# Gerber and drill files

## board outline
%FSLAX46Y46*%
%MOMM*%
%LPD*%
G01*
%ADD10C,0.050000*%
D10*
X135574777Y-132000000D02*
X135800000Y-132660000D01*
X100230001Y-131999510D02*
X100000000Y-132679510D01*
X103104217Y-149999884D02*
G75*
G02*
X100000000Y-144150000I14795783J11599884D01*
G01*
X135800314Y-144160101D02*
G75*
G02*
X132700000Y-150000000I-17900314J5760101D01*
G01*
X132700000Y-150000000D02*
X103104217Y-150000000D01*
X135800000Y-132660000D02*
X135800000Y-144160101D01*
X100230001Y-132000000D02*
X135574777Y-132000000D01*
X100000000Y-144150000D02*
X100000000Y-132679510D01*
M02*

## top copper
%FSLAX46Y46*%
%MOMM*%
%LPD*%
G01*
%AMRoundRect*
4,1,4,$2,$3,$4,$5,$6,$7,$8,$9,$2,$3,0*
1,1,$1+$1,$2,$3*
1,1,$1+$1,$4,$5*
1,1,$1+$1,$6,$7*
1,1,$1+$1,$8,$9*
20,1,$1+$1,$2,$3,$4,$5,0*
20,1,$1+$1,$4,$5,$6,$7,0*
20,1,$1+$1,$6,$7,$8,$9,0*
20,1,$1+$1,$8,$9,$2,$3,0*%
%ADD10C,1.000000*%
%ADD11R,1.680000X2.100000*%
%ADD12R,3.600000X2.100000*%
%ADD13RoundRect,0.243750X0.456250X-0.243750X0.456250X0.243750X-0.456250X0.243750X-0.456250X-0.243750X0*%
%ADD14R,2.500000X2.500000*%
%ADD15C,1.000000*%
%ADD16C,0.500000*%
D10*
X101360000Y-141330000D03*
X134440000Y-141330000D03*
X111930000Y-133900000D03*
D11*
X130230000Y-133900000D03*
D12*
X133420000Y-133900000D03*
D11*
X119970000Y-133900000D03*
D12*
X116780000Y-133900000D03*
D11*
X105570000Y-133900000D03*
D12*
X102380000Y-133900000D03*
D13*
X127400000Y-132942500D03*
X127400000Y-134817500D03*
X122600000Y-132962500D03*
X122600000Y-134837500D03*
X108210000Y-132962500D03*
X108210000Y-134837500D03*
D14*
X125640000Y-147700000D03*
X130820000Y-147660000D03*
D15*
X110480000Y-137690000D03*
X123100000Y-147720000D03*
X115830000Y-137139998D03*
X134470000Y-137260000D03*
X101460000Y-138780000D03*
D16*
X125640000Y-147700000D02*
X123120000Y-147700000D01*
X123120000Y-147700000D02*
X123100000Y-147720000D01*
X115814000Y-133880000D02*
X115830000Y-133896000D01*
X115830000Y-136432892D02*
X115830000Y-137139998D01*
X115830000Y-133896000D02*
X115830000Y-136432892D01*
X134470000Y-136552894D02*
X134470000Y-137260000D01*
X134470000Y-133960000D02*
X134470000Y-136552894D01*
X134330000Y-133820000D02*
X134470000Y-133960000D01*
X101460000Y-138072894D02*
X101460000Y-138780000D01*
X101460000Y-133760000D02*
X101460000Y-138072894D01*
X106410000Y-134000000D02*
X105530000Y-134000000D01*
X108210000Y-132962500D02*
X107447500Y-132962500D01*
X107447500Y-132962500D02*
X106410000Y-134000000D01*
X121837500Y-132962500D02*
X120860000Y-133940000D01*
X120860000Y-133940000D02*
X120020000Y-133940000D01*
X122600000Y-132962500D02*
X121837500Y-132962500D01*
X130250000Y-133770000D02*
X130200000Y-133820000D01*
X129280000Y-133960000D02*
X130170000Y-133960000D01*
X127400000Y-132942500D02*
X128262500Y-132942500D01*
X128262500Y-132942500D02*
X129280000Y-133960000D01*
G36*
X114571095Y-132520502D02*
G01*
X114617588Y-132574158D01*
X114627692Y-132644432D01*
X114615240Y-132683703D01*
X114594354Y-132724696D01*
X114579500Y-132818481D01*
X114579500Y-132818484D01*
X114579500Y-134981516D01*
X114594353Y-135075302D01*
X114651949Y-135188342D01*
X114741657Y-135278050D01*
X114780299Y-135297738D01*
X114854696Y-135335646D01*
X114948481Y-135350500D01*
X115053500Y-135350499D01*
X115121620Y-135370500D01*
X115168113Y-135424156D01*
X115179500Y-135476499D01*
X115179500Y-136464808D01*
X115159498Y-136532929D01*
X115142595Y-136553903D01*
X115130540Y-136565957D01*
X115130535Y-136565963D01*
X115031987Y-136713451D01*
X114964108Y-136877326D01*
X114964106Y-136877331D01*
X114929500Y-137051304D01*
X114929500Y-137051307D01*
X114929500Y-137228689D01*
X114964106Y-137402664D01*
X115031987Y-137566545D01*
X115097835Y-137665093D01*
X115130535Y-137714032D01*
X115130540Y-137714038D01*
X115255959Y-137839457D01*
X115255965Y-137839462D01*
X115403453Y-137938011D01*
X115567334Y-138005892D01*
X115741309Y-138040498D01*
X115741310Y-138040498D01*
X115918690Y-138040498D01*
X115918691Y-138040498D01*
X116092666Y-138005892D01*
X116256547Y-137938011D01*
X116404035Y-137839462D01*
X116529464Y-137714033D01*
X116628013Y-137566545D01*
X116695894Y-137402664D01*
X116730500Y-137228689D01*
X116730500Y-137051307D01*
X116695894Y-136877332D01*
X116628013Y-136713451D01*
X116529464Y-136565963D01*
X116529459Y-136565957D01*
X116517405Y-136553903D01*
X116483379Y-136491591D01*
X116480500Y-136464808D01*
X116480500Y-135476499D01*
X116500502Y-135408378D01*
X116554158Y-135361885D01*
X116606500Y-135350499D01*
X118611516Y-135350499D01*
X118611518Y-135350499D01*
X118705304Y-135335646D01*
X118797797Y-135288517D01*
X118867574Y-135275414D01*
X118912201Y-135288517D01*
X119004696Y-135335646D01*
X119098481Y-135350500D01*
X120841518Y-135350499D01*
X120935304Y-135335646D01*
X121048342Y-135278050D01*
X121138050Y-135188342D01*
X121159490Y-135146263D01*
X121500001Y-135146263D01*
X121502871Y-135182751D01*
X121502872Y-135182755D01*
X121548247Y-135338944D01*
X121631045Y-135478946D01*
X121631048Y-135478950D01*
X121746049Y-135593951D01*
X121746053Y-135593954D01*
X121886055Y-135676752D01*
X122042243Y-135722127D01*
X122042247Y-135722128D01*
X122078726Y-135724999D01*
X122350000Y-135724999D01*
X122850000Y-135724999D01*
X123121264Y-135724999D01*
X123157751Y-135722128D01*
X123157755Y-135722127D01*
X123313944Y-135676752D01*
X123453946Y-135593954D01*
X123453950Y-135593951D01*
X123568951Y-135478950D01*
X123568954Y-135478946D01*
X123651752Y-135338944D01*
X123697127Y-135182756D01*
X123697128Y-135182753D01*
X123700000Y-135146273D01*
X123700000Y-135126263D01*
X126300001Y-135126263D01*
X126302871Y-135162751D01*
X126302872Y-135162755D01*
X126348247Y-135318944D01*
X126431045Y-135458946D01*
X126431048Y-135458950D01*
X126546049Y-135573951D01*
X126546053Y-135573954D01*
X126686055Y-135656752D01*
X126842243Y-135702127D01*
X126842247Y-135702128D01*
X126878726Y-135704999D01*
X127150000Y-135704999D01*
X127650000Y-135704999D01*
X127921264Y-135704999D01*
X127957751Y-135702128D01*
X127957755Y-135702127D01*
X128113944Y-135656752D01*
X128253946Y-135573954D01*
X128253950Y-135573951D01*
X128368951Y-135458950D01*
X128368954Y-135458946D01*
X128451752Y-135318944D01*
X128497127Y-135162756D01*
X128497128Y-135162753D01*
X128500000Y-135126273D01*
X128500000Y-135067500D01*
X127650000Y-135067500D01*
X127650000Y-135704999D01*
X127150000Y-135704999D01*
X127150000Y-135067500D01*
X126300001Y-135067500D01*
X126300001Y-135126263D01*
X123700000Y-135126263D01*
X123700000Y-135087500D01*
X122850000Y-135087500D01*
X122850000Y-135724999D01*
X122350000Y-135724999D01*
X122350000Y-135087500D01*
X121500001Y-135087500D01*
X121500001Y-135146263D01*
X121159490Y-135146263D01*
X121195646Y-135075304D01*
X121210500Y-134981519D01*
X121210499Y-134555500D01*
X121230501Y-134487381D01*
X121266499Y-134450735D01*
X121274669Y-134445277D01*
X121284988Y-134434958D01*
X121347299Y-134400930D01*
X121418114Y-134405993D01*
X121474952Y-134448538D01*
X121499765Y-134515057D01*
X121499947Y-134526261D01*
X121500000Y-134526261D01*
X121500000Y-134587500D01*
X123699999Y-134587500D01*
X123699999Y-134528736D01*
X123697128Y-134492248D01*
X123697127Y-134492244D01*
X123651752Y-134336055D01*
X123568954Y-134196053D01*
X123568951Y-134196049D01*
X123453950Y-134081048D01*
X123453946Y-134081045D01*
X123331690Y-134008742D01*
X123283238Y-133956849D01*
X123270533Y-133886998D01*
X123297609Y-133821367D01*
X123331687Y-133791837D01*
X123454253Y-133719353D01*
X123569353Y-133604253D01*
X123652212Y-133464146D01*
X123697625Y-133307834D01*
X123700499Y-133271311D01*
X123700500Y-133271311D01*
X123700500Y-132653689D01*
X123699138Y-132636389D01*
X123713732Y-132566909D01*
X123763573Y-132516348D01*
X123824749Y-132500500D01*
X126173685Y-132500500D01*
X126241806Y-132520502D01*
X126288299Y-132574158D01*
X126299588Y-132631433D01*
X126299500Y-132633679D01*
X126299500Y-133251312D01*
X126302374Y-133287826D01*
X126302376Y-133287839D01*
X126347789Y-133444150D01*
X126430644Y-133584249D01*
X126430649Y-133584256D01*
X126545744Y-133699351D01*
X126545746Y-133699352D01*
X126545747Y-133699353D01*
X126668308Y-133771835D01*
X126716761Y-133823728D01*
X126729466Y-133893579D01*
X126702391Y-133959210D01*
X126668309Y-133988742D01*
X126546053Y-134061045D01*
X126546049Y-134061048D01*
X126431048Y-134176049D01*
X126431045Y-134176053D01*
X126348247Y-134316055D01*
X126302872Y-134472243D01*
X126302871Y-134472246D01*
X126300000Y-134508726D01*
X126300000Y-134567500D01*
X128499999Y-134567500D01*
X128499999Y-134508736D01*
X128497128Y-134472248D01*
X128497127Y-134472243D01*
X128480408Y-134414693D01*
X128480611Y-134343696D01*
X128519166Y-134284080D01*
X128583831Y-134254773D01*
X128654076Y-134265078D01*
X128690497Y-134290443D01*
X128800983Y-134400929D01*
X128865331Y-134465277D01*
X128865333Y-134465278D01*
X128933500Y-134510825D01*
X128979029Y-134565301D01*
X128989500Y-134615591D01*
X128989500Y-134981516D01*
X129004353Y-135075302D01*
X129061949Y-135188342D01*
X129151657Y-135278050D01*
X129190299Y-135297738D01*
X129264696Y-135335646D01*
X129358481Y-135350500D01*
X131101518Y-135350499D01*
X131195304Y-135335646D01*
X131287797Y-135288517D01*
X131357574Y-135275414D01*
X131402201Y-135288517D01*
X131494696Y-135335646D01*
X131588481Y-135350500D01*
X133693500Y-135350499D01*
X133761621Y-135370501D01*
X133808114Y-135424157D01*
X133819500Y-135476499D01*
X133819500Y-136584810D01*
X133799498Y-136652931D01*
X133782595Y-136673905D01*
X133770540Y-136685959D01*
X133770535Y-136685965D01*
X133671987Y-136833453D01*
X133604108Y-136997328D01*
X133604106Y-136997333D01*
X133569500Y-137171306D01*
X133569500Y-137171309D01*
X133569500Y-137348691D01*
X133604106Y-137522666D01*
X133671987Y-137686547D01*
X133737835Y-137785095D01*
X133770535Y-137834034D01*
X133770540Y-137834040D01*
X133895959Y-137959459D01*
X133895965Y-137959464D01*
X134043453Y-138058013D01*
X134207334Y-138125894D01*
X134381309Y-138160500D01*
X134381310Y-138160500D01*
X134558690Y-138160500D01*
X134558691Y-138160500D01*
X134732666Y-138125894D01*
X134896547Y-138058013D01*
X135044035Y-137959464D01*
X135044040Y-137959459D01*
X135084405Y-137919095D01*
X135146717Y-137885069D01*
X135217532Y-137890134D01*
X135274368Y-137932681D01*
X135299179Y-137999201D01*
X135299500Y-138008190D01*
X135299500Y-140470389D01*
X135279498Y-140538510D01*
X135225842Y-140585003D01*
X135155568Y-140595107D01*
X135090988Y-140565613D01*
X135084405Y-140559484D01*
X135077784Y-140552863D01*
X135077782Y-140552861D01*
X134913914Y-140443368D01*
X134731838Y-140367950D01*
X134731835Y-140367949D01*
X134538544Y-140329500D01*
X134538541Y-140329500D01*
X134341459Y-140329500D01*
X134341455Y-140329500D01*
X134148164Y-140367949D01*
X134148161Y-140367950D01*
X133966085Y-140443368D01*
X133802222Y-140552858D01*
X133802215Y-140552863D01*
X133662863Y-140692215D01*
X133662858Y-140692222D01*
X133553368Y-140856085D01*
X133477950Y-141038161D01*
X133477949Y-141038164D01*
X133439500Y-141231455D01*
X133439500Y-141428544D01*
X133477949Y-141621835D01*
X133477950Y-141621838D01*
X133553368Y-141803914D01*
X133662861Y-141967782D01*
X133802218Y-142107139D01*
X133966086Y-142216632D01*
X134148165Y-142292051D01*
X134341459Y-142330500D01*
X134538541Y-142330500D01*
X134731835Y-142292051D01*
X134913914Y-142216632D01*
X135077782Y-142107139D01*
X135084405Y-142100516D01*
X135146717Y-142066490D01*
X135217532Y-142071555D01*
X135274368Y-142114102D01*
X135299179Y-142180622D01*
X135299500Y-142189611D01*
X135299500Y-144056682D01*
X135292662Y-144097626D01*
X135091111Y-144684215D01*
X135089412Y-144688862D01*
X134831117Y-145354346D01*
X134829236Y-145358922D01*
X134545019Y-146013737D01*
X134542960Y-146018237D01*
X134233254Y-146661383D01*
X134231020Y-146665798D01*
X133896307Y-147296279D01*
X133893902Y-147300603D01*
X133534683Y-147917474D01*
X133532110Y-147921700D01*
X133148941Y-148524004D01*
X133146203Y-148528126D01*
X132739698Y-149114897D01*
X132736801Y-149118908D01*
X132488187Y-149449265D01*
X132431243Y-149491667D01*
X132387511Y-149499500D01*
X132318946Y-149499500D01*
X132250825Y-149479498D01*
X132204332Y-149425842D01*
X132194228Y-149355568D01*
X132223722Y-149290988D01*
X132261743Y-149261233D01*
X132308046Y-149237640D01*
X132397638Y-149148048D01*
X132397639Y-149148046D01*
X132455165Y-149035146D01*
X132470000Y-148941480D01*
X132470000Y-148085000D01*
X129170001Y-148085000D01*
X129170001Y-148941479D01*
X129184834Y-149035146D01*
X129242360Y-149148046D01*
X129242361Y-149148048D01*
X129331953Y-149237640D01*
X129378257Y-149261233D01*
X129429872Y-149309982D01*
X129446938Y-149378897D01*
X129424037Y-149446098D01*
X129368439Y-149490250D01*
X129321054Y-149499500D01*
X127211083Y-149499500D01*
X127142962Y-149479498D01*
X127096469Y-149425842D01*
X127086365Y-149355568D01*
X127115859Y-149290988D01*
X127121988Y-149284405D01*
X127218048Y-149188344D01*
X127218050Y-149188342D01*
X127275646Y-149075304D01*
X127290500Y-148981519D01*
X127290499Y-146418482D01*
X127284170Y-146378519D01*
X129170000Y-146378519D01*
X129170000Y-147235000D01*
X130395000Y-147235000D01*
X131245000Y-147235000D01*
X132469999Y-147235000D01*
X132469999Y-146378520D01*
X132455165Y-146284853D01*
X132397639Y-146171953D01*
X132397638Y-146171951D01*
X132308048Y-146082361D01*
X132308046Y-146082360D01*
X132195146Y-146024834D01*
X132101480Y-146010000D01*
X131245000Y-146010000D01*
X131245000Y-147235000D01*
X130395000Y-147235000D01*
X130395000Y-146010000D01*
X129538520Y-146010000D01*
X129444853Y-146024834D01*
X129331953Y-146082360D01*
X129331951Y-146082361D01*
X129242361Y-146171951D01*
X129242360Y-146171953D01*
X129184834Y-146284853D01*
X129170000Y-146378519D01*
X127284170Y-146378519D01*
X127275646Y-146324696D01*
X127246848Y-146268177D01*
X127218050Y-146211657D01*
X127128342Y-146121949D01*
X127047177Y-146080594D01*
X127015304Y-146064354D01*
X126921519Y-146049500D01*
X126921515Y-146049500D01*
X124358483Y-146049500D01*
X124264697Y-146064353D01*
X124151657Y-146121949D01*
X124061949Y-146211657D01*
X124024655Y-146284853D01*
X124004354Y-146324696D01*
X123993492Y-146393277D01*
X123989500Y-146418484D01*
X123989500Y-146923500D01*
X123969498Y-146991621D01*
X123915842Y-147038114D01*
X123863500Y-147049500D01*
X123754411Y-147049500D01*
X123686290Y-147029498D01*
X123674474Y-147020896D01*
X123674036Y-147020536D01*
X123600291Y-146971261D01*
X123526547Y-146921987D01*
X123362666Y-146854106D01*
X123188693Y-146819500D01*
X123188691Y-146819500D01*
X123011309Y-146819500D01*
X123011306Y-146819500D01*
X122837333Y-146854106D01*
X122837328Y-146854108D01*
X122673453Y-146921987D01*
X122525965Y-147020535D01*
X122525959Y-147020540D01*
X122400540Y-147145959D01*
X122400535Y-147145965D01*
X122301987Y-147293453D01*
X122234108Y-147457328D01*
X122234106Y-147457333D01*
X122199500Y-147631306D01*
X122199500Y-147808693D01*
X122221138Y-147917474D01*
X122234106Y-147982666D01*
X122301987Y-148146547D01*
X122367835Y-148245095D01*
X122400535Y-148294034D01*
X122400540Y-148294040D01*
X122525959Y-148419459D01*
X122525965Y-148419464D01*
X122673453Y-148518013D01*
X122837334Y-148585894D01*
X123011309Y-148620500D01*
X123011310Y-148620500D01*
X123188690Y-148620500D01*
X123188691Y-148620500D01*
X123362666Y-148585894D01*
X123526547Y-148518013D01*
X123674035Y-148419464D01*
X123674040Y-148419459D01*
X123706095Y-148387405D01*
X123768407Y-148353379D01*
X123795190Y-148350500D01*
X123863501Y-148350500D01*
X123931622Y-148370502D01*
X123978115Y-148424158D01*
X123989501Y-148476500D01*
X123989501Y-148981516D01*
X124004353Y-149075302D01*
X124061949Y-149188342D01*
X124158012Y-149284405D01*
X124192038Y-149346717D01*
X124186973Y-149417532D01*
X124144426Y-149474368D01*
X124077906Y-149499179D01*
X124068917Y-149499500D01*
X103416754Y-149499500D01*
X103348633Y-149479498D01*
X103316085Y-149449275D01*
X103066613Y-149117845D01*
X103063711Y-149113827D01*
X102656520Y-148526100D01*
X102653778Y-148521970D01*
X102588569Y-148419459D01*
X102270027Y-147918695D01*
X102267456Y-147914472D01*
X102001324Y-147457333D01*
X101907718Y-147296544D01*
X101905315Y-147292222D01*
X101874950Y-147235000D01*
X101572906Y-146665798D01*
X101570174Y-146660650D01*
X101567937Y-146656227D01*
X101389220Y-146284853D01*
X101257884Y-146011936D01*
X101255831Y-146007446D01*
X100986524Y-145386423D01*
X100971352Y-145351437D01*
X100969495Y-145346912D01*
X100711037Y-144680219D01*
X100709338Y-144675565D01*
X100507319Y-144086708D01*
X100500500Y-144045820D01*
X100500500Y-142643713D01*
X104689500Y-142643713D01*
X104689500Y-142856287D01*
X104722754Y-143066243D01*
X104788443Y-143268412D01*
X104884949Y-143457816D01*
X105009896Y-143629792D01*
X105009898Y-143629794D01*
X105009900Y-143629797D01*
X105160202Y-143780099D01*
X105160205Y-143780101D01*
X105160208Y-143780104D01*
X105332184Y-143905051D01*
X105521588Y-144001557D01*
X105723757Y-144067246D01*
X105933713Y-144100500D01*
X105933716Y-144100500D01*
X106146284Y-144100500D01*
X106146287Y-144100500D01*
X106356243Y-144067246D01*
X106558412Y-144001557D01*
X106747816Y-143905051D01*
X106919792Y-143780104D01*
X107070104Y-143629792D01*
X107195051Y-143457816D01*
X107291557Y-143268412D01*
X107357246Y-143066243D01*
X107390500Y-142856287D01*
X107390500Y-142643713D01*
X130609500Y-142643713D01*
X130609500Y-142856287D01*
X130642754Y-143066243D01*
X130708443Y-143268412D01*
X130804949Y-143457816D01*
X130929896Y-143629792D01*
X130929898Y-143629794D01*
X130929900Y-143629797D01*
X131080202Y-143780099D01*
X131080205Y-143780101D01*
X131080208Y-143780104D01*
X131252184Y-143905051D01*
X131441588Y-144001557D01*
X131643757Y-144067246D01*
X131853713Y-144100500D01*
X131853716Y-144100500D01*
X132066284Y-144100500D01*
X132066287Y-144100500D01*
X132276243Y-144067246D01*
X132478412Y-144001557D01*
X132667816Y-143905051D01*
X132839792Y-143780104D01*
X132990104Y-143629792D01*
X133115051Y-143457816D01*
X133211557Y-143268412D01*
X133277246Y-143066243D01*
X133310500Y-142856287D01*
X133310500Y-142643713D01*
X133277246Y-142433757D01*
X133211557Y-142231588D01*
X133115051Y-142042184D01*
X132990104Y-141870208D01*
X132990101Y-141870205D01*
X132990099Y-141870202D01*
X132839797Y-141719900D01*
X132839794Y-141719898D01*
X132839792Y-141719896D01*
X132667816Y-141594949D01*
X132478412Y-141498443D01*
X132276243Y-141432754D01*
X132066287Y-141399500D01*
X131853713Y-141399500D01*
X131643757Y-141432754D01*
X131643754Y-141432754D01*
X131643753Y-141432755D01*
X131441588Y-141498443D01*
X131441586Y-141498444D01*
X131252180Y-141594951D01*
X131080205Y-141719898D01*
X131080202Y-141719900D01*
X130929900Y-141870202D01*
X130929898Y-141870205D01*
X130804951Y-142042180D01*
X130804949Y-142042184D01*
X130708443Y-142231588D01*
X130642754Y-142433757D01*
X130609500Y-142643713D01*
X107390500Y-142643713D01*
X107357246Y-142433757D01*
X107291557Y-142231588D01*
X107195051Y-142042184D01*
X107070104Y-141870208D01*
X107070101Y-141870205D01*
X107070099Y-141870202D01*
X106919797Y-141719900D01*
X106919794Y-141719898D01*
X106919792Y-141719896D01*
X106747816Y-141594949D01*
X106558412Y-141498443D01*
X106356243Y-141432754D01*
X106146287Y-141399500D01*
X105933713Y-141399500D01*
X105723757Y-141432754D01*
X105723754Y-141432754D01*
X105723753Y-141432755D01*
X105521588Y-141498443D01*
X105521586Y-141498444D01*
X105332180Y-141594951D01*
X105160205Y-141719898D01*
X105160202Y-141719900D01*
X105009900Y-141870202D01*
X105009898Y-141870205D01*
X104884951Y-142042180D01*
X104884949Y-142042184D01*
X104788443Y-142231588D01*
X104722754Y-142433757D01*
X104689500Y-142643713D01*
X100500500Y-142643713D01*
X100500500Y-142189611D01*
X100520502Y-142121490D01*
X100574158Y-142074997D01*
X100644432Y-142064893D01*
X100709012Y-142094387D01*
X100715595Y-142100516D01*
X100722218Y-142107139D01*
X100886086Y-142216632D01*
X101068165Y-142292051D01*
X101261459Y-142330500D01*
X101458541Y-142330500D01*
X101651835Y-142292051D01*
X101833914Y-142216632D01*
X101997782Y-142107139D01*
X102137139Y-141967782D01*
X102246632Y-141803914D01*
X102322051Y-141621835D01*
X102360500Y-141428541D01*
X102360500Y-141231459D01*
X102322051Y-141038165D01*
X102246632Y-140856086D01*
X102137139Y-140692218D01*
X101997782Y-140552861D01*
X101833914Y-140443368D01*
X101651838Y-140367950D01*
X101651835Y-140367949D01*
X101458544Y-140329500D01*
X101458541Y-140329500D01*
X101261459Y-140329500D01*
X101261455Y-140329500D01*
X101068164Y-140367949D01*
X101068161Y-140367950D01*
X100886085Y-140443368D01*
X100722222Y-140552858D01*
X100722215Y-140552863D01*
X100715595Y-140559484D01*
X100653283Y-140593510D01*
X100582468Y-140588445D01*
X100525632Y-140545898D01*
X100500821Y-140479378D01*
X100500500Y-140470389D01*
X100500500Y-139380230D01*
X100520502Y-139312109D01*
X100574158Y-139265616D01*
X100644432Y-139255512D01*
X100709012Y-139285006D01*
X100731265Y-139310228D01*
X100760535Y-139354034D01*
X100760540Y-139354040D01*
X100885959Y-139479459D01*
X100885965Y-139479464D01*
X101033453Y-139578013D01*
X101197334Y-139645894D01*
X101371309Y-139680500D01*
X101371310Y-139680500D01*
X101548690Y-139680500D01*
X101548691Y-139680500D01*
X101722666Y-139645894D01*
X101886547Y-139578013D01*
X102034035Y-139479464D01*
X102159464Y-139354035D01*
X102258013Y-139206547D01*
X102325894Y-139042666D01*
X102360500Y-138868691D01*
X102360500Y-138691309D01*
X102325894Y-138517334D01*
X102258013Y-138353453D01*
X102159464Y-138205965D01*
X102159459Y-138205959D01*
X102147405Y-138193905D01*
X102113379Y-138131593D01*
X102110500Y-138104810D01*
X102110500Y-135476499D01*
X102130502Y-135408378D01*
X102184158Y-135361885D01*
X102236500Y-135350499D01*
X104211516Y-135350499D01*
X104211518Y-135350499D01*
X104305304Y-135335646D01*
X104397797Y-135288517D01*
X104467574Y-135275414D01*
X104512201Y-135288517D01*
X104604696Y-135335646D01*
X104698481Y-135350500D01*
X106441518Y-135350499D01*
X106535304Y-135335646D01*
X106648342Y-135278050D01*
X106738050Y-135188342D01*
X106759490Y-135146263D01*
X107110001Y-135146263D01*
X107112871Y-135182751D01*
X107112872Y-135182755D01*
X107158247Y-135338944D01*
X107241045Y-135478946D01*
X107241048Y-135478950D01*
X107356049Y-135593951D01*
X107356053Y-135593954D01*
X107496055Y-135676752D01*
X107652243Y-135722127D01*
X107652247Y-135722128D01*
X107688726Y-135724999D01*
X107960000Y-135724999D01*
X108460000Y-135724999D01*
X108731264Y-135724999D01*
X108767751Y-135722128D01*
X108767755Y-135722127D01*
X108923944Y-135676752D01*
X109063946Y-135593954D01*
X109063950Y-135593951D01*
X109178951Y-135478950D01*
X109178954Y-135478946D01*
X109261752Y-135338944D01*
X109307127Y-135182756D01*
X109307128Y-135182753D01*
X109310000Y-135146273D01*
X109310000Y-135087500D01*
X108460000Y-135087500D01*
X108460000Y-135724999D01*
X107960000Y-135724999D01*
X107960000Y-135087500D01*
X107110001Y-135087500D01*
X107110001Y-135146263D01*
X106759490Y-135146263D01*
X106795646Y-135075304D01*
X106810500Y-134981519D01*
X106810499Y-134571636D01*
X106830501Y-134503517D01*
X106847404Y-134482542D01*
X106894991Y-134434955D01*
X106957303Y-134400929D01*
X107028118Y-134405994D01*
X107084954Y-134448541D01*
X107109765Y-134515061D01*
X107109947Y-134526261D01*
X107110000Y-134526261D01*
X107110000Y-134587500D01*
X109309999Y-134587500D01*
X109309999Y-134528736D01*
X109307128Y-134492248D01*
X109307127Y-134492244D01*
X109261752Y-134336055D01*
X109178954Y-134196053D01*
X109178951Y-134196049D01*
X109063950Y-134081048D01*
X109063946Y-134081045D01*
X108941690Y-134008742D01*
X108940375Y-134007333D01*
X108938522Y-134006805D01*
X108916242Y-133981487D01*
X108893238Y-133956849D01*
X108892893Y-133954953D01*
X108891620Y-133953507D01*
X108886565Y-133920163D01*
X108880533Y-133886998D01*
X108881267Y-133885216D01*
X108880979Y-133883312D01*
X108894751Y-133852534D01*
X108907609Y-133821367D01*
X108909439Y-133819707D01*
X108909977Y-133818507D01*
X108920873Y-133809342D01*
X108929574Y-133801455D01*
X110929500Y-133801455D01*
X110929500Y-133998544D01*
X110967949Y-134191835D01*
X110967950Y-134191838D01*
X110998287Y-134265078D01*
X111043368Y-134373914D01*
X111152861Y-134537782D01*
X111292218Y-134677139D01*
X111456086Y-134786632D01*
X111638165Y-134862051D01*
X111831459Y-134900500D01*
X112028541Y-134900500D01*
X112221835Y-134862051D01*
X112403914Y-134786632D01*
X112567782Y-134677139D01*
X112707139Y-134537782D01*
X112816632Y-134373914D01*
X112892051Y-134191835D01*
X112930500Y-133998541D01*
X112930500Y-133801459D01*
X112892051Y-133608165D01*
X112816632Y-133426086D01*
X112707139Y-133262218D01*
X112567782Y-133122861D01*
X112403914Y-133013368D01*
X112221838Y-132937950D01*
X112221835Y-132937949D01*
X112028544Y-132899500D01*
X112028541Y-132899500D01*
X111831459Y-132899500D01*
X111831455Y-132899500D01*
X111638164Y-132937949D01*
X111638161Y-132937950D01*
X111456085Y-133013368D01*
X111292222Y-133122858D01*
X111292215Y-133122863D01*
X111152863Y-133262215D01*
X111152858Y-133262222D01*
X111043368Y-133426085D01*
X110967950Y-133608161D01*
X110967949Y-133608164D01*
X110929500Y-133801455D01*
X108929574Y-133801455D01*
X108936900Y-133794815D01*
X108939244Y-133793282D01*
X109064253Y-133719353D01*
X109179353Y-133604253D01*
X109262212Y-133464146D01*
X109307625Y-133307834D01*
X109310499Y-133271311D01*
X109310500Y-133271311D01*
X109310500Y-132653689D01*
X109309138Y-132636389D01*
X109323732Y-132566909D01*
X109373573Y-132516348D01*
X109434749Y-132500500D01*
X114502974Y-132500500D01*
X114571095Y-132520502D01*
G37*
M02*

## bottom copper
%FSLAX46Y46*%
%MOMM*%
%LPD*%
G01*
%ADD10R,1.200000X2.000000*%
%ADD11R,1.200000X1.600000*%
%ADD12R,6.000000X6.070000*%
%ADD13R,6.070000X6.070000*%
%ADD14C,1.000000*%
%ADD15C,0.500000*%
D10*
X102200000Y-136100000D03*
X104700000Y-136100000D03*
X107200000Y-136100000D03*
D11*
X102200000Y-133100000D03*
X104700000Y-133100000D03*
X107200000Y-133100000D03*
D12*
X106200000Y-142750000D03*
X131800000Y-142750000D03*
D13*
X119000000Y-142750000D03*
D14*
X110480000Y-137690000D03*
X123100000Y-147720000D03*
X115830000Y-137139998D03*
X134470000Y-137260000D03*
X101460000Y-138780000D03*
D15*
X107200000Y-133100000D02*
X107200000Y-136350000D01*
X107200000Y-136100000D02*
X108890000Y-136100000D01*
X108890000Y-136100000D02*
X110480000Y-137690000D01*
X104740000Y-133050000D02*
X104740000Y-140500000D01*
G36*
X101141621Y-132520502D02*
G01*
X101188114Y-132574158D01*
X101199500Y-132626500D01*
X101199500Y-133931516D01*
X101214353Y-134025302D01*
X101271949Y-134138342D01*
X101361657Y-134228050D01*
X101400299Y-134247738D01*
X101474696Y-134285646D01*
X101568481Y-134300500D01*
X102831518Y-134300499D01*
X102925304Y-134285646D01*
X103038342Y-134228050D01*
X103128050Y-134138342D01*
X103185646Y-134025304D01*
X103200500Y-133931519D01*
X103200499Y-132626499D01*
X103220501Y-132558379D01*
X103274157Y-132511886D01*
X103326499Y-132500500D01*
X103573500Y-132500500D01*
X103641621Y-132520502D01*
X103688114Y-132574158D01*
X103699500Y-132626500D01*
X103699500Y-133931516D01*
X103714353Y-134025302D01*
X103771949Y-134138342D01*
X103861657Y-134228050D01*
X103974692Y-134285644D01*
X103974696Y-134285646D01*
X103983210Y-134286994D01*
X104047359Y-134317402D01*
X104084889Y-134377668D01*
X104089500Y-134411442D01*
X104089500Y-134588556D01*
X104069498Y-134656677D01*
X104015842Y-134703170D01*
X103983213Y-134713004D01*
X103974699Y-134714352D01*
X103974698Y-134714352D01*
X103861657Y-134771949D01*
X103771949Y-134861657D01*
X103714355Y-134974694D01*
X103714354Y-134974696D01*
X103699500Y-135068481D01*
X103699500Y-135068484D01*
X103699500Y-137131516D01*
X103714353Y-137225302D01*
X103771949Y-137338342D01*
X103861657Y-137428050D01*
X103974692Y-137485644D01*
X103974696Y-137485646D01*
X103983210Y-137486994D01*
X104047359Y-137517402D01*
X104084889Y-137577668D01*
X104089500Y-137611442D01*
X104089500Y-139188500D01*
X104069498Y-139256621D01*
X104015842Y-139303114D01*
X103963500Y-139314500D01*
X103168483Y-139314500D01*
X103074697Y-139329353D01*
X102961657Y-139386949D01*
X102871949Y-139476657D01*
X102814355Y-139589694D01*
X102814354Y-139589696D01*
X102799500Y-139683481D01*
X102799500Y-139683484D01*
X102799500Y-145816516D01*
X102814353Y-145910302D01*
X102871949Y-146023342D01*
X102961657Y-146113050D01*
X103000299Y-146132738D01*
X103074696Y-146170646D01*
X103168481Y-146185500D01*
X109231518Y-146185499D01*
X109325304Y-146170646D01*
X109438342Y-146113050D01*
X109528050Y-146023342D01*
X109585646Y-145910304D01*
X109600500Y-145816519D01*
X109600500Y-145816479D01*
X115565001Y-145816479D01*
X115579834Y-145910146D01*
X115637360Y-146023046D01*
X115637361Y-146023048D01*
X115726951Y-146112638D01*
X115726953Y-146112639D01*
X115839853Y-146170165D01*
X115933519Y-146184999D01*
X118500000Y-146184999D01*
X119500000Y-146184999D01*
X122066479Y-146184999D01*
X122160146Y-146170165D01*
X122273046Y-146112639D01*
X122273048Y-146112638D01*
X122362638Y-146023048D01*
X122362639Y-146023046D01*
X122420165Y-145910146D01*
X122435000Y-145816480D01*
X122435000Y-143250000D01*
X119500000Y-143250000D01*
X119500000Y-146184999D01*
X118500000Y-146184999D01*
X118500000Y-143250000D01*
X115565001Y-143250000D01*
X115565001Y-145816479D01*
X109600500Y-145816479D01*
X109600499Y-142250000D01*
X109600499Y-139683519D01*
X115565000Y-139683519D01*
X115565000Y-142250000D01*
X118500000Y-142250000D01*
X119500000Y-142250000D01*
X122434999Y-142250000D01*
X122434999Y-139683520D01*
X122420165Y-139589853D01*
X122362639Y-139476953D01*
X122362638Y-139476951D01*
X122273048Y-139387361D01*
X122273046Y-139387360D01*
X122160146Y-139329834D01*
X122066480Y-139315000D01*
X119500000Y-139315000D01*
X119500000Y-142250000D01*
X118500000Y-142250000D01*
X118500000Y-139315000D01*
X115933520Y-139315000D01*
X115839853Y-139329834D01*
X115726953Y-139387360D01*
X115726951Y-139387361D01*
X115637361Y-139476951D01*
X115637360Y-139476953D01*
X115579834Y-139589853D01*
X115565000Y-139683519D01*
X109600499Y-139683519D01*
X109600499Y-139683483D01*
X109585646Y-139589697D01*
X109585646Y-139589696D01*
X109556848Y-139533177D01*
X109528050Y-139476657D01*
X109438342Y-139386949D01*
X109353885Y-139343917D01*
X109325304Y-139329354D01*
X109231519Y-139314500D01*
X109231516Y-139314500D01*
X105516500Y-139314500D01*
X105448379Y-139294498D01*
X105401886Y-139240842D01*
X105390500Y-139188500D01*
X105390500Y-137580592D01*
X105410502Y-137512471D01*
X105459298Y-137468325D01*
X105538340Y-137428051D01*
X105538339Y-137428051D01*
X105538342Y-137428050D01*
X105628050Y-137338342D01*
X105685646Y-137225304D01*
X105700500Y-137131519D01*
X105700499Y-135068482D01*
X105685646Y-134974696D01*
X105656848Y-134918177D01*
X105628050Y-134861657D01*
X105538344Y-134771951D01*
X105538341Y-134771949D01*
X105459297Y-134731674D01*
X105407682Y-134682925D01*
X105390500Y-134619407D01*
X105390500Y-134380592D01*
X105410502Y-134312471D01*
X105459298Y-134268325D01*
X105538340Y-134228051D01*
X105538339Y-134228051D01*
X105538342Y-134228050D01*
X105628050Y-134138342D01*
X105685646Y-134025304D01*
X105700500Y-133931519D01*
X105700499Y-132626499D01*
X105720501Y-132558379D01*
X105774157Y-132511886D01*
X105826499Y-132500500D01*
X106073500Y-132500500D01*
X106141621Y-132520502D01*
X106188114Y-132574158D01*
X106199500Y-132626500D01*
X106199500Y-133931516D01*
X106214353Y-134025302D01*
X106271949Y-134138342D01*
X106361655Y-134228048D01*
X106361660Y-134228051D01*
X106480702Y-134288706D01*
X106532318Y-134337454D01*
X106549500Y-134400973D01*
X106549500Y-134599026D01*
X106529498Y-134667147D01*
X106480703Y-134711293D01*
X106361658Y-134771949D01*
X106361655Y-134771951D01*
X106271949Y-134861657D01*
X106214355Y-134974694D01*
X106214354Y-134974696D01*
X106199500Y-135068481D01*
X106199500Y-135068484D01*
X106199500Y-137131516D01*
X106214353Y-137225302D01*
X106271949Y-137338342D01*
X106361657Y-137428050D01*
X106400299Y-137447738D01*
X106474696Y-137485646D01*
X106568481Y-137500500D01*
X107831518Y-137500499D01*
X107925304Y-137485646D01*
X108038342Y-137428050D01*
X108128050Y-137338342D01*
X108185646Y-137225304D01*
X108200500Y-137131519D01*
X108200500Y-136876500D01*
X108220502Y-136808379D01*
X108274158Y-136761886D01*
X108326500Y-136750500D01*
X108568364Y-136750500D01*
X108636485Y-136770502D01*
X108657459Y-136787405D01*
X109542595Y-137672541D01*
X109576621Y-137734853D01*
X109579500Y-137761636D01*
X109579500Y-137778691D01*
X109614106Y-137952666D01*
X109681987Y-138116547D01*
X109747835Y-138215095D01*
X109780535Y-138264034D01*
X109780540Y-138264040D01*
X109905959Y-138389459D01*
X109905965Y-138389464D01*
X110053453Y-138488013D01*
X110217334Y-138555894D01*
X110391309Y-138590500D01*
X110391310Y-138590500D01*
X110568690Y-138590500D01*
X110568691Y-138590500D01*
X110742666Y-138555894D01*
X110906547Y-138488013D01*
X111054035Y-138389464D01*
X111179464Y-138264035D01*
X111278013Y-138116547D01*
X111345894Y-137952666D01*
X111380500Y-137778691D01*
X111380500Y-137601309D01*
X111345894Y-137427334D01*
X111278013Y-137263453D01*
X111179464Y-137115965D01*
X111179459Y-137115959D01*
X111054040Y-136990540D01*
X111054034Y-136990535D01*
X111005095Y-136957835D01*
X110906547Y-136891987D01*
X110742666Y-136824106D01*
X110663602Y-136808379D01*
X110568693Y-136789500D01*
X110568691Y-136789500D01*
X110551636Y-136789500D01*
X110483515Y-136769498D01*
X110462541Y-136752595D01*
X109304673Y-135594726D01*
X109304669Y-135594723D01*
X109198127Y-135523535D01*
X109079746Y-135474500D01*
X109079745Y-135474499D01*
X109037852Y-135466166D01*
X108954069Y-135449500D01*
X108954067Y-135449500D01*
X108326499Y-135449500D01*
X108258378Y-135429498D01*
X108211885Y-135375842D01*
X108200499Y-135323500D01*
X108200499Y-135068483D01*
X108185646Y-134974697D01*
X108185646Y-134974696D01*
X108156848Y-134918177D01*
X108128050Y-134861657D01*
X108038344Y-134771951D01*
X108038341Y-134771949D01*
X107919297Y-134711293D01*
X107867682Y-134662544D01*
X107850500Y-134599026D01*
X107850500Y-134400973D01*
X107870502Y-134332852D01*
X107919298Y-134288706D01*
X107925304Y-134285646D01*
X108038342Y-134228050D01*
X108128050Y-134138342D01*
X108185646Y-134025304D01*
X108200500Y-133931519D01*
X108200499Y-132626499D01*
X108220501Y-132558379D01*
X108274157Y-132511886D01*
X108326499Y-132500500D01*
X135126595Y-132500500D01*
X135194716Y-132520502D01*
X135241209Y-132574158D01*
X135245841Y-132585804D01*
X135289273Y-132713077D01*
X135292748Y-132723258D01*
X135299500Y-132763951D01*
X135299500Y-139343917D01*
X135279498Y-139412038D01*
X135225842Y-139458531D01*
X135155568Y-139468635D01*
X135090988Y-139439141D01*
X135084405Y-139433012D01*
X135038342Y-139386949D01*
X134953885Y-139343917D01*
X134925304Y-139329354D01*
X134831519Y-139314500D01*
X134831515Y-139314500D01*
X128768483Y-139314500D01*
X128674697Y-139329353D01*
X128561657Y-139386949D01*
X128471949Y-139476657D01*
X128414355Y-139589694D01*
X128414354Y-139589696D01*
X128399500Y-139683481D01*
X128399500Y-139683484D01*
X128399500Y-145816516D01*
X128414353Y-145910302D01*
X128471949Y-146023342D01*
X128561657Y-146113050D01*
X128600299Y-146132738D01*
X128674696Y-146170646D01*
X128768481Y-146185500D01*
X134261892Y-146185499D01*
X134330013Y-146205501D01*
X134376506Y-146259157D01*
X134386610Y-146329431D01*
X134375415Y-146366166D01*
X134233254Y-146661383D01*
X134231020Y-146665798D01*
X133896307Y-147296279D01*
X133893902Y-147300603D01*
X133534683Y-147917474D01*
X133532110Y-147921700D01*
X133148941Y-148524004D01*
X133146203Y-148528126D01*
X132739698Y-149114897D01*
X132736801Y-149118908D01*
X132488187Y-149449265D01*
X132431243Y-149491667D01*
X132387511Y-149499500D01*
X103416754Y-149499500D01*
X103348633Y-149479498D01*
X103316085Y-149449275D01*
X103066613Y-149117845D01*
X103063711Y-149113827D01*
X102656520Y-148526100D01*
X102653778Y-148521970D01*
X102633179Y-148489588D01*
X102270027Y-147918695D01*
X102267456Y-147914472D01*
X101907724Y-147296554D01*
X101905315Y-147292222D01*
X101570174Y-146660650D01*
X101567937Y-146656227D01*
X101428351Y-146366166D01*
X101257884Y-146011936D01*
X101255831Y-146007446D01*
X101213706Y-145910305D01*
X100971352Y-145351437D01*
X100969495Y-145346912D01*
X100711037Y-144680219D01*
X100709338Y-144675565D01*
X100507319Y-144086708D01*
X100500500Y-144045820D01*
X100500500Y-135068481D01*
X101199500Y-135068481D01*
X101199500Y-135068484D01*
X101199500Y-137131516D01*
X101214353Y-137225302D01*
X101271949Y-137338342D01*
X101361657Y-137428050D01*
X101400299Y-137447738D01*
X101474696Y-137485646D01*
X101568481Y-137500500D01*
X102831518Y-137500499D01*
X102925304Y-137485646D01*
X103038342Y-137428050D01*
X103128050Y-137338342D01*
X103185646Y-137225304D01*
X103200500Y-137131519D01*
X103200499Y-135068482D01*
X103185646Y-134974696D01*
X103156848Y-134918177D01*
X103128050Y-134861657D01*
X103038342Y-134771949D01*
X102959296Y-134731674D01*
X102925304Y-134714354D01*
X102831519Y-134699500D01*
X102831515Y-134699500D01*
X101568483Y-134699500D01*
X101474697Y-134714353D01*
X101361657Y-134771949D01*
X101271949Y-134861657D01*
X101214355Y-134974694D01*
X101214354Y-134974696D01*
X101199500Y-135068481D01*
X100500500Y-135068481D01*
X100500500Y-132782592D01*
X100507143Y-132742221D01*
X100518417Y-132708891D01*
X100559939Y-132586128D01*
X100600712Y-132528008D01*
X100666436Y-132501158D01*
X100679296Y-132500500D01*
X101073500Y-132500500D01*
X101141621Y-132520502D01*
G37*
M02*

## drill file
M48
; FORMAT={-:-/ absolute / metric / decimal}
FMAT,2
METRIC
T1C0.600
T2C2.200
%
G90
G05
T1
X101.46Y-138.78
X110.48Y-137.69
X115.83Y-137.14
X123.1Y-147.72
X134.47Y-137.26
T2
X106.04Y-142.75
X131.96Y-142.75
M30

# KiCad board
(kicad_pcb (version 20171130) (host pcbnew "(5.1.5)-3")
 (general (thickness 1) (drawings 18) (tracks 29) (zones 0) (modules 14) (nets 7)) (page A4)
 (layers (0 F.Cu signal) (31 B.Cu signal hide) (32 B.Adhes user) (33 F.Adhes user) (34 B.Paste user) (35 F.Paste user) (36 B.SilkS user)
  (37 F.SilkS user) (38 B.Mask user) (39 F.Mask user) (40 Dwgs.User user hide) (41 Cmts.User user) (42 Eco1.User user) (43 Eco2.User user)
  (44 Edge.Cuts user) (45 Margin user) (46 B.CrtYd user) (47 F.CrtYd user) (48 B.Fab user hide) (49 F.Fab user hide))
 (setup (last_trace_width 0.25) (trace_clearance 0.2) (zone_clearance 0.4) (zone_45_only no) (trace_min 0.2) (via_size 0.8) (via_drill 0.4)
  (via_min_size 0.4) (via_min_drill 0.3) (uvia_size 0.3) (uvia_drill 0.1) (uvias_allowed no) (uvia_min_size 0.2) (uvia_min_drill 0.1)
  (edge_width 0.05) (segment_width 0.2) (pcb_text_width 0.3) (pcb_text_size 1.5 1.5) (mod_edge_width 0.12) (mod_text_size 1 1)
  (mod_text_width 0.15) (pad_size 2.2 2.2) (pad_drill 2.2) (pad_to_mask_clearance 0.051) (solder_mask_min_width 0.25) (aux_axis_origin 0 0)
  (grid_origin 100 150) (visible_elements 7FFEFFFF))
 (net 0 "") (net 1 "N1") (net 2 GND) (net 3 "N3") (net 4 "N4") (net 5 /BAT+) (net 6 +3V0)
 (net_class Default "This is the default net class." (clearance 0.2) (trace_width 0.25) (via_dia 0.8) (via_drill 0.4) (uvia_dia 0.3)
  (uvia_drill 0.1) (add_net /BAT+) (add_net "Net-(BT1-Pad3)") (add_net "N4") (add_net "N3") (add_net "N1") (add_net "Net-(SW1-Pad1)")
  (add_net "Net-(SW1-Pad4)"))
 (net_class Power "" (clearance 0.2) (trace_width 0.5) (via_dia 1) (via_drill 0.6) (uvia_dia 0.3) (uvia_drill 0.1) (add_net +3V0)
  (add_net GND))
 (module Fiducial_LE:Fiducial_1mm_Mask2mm (layer F.Cu) (at 101.36 141.33)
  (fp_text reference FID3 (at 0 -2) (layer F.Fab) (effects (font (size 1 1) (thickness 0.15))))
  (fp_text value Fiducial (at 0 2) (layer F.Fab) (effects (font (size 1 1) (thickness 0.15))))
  (pad "" smd circle (at 0 0) (size 1 1) (layers F.Cu F.Mask) (solder_mask_margin 0.5) (clearance 0.5)))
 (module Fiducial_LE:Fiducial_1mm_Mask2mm (layer F.Cu) (at 134.44 141.33)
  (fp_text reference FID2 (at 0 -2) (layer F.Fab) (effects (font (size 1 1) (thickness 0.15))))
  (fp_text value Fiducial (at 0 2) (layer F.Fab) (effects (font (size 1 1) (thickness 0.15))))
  (pad "" smd circle (at 0 0) (size 1 1) (layers F.Cu F.Mask) (solder_mask_margin 0.5) (clearance 0.5)))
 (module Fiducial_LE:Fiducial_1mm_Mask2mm (layer F.Cu) (at 111.93 133.9)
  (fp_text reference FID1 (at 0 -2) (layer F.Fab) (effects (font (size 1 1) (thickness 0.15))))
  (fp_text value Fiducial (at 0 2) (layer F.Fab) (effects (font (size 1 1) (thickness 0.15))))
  (pad "" smd circle (at 0 0) (size 1 1) (layers F.Cu F.Mask) (solder_mask_margin 0.5) (clearance 0.5)))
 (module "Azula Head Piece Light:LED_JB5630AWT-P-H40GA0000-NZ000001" (layer F.Cu) (at 132.3 133.9 180)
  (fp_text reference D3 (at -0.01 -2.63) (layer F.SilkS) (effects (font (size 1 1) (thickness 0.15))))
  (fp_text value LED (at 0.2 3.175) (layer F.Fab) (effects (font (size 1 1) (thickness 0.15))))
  (pad 2 smd rect (at 2.07 0 90) (size 2.1 1.68) (layers F.Cu F.Paste F.Mask) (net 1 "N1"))
  (pad 1 smd rect (at -1.12 0) (size 3.6 2.1) (layers F.Cu F.Paste F.Mask) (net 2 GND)))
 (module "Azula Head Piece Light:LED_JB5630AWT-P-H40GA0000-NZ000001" (layer F.Cu) (at 117.9 133.9)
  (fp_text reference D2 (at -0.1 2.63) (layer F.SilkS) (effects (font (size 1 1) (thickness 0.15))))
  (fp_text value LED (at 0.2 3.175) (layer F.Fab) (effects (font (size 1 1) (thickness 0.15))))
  (pad 2 smd rect (at 2.07 0 270) (size 2.1 1.68) (layers F.Cu F.Paste F.Mask) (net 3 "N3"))
  (pad 1 smd rect (at -1.12 0 180) (size 3.6 2.1) (layers F.Cu F.Paste F.Mask) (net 2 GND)))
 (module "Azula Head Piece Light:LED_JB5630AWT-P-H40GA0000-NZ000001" (layer F.Cu) (at 103.5 133.9)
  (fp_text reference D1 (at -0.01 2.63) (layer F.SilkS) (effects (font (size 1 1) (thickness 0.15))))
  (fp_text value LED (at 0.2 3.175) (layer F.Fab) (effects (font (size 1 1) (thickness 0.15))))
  (pad 2 smd rect (at 2.07 0 270) (size 2.1 1.68) (layers F.Cu F.Paste F.Mask) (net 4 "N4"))
  (pad 1 smd rect (at -1.12 0 180) (size 3.6 2.1) (layers F.Cu F.Paste F.Mask) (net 2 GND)))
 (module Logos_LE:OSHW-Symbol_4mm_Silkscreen (layer F.Cu) (at 117.894157 141.33)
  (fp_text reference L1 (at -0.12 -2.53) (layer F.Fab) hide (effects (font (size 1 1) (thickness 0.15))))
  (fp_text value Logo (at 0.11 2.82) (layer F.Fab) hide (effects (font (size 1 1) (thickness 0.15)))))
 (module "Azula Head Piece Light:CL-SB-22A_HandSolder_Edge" (layer B.Cu) (at 104.7 134.5)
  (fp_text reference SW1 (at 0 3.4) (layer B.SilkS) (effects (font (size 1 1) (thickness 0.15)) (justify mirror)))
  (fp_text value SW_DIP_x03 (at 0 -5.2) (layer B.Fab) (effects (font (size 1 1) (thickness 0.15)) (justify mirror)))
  (pad 4 smd rect (at -2.5 1.6) (size 1.2 2) (layers B.Cu B.Paste B.Mask))
  (pad 5 smd rect (at 0 1.6) (size 1.2 2) (layers B.Cu B.Paste B.Mask) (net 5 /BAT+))
  (pad 6 smd rect (at 2.5 1.6) (size 1.2 2) (layers B.Cu B.Paste B.Mask) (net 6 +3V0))
  (pad 1 smd rect (at -2.5 -1.4) (size 1.2 1.6) (layers B.Cu B.Paste B.Mask))
  (pad 2 smd rect (at 0 -1.4) (size 1.2 1.6) (layers B.Cu B.Paste B.Mask) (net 5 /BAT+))
  (pad 3 smd rect (at 2.5 -1.4) (size 1.2 1.6) (layers B.Cu B.Paste B.Mask) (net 6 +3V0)))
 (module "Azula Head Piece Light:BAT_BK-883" (layer B.Cu) (at 119 142.75)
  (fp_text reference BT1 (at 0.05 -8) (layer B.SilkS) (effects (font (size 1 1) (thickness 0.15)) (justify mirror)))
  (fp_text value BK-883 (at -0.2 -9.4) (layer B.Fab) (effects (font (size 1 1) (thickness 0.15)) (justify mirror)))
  (pad "" np_thru_hole circle (at -12.96 0) (size 2.2 2.2) (drill 2.2) (layers *.Cu *.Mask))
  (pad "" np_thru_hole circle (at 12.96 0) (size 2.2 2.2) (drill 2.2) (layers *.Cu *.Mask))
  (pad 1 smd rect (at -12.8 0) (size 6 6.07) (layers B.Cu B.Paste B.Mask) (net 5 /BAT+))
  (pad 3 smd rect (at 12.8 0) (size 6 6.07) (layers B.Cu B.Paste B.Mask))
  (pad 2 smd rect (at 0 0) (size 6.07 6.07) (layers B.Cu B.Paste B.Mask) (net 2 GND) (thermal_width 1)))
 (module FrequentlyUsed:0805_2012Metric (layer F.Cu) (at 127.4 133.88 90)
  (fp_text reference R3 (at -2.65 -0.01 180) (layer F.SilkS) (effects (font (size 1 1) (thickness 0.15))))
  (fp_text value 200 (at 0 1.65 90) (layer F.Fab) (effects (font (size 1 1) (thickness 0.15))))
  (pad 2 smd roundrect (at 0.9375 0 90) (size 0.975 1.4) (layers F.Cu F.Paste F.Mask) (roundrect_rratio 0.25) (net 1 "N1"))
  (pad 1 smd roundrect (at -0.9375 0 90) (size 0.975 1.4) (layers F.Cu F.Paste F.Mask) (roundrect_rratio 0.25) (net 6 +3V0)))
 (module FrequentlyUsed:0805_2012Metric (layer F.Cu) (at 122.6 133.9 90)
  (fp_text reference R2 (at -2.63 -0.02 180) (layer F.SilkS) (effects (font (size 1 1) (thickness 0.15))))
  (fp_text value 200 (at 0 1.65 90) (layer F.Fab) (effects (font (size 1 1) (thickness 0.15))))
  (pad 2 smd roundrect (at 0.9375 0 90) (size 0.975 1.4) (layers F.Cu F.Paste F.Mask) (roundrect_rratio 0.25) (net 3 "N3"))
  (pad 1 smd roundrect (at -0.9375 0 90) (size 0.975 1.4) (layers F.Cu F.Paste F.Mask) (roundrect_rratio 0.25) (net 6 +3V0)))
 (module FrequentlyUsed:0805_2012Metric (layer F.Cu) (at 108.21 133.9 90)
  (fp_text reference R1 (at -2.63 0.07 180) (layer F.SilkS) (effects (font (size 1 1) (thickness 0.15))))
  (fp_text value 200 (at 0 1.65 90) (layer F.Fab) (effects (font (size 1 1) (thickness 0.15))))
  (pad 2 smd roundrect (at 0.9375 0 90) (size 0.975 1.4) (layers F.Cu F.Paste F.Mask) (roundrect_rratio 0.25) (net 4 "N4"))
  (pad 1 smd roundrect (at -0.9375 0 90) (size 0.975 1.4) (layers F.Cu F.Paste F.Mask) (roundrect_rratio 0.25) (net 6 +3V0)))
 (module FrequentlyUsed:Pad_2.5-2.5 (layer F.Cu) (at 125.64 147.7)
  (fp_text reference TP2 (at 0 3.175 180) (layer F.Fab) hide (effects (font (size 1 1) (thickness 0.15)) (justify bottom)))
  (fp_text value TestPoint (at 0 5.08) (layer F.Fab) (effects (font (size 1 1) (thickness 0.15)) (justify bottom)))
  (pad 1 smd rect (at 0 0) (size 2.5 2.5) (layers F.Cu F.Mask) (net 2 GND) (solder_mask_margin 0.1016) (thermal_width 0.85)))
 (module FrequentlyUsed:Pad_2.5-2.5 (layer F.Cu) (at 130.82 147.66)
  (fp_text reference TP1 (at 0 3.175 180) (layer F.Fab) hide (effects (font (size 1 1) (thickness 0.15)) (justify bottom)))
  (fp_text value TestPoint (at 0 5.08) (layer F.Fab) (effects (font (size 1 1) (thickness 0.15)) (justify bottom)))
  (pad 1 smd rect (at 0 0) (size 2.5 2.5) (layers F.Cu F.Mask) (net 6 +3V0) (solder_mask_margin 0.1016) (thermal_width 0.85)))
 (gr_line (start 135.574777 132) (end 135.8 132.66) (layer Edge.Cuts) (width 0.05))
 (gr_line (start 100.230001 131.99951) (end 100 132.67951) (layer Edge.Cuts) (width 0.05))
 (gr_arc (start 117.9 138.4) (end 100 144.15) (angle -20.28789713) (layer Edge.Cuts) (width 0.05))
 (gr_arc (start 117.9 138.4) (end 132.7 150) (angle -20.25123582) (layer Edge.Cuts) (width 0.05))
 (gr_line (start 132.7 150) (end 103.104217 150) (layer Edge.Cuts) (width 0.05))
 (gr_line (start 135.8 132.66) (end 135.8 144.160101) (layer Edge.Cuts) (width 0.05))
 (gr_line (start 100.230001 132) (end 135.574777 132) (layer Edge.Cuts) (width 0.05))
 (gr_line (start 100 144.15) (end 100 132.67951) (layer Edge.Cuts) (width 0.05))
 (segment (start 107.2 133.1) (end 107.2 136.35) (width 0.5) (layer B.Cu) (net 6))
 (via (at 110.48 137.69) (size 1) (drill 0.6) (layers F.Cu B.Cu) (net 6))
 (segment (start 107.2 136.1) (end 108.89 136.1) (width 0.5) (layer B.Cu) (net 6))
 (segment (start 108.89 136.1) (end 110.48 137.69) (width 0.5) (layer B.Cu) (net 6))
 (via (at 123.1 147.72) (size 1) (drill 0.6) (layers F.Cu B.Cu) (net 2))
 (segment (start 125.64 147.7) (end 123.12 147.7) (width 0.5) (layer F.Cu) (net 2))
 (segment (start 123.12 147.7) (end 123.1 147.72) (width 0.5) (layer F.Cu) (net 2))
 (via (at 115.83 137.139998) (size 1) (drill 0.6) (layers F.Cu B.Cu) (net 2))
 (segment (start 115.814 133.88) (end 115.83 133.896) (width 0.5) (layer F.Cu) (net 2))
 (segment (start 115.83 136.432892) (end 115.83 137.139998) (width 0.5) (layer F.Cu) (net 2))
 (segment (start 115.83 133.896) (end 115.83 136.432892) (width 0.5) (layer F.Cu) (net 2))
 (via (at 134.47 137.26) (size 1) (drill 0.6) (layers F.Cu B.Cu) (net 2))
 (segment (start 134.47 136.552894) (end 134.47 137.26) (width 0.5) (layer F.Cu) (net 2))
 (segment (start 134.47 133.96) (end 134.47 136.552894) (width 0.5) (layer F.Cu) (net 2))
 (segment (start 134.33 133.82) (end 134.47 133.96) (width 0.5) (layer F.Cu) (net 2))
 (via (at 101.46 138.78) (size 1) (drill 0.6) (layers F.Cu B.Cu) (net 2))
 (segment (start 101.46 138.072894) (end 101.46 138.78) (width 0.5) (layer F.Cu) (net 2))
 (segment (start 101.46 133.76) (end 101.46 138.072894) (width 0.5) (layer F.Cu) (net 2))
 (segment (start 104.74 133.05) (end 104.74 140.5) (width 0.5) (layer B.Cu) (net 5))
 (segment (start 106.41 134) (end 105.53 134) (width 0.5) (layer F.Cu) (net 4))
 (segment (start 108.21 132.9625) (end 107.4475 132.9625) (width 0.5) (layer F.Cu) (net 4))
 (segment (start 107.4475 132.9625) (end 106.41 134) (width 0.5) (layer F.Cu) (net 4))
 (segment (start 121.8375 132.9625) (end 120.86 133.94) (width 0.5) (layer F.Cu) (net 3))
 (segment (start 120.86 133.94) (end 120.02 133.94) (width 0.5) (layer F.Cu) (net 3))
 (segment (start 122.6 132.9625) (end 121.8375 132.9625) (width 0.5) (layer F.Cu) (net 3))
 (segment (start 130.25 133.77) (end 130.2 133.82) (width 0.5) (layer F.Cu) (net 1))
 (segment (start 129.28 133.96) (end 130.17 133.96) (width 0.5) (layer F.Cu) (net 1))
 (segment (start 127.4 132.9425) (end 128.2625 132.9425) (width 0.5) (layer F.Cu) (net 1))
 (segment (start 128.2625 132.9425) (end 129.28 133.96) (width 0.5) (layer F.Cu) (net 1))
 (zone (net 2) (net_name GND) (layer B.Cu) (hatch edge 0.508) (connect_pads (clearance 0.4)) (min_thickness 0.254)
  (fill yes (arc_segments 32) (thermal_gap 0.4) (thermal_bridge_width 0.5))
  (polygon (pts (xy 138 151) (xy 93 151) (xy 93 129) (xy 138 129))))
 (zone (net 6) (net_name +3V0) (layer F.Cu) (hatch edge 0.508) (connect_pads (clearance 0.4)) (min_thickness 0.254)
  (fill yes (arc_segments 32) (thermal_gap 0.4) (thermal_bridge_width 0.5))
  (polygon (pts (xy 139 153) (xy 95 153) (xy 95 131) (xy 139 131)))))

